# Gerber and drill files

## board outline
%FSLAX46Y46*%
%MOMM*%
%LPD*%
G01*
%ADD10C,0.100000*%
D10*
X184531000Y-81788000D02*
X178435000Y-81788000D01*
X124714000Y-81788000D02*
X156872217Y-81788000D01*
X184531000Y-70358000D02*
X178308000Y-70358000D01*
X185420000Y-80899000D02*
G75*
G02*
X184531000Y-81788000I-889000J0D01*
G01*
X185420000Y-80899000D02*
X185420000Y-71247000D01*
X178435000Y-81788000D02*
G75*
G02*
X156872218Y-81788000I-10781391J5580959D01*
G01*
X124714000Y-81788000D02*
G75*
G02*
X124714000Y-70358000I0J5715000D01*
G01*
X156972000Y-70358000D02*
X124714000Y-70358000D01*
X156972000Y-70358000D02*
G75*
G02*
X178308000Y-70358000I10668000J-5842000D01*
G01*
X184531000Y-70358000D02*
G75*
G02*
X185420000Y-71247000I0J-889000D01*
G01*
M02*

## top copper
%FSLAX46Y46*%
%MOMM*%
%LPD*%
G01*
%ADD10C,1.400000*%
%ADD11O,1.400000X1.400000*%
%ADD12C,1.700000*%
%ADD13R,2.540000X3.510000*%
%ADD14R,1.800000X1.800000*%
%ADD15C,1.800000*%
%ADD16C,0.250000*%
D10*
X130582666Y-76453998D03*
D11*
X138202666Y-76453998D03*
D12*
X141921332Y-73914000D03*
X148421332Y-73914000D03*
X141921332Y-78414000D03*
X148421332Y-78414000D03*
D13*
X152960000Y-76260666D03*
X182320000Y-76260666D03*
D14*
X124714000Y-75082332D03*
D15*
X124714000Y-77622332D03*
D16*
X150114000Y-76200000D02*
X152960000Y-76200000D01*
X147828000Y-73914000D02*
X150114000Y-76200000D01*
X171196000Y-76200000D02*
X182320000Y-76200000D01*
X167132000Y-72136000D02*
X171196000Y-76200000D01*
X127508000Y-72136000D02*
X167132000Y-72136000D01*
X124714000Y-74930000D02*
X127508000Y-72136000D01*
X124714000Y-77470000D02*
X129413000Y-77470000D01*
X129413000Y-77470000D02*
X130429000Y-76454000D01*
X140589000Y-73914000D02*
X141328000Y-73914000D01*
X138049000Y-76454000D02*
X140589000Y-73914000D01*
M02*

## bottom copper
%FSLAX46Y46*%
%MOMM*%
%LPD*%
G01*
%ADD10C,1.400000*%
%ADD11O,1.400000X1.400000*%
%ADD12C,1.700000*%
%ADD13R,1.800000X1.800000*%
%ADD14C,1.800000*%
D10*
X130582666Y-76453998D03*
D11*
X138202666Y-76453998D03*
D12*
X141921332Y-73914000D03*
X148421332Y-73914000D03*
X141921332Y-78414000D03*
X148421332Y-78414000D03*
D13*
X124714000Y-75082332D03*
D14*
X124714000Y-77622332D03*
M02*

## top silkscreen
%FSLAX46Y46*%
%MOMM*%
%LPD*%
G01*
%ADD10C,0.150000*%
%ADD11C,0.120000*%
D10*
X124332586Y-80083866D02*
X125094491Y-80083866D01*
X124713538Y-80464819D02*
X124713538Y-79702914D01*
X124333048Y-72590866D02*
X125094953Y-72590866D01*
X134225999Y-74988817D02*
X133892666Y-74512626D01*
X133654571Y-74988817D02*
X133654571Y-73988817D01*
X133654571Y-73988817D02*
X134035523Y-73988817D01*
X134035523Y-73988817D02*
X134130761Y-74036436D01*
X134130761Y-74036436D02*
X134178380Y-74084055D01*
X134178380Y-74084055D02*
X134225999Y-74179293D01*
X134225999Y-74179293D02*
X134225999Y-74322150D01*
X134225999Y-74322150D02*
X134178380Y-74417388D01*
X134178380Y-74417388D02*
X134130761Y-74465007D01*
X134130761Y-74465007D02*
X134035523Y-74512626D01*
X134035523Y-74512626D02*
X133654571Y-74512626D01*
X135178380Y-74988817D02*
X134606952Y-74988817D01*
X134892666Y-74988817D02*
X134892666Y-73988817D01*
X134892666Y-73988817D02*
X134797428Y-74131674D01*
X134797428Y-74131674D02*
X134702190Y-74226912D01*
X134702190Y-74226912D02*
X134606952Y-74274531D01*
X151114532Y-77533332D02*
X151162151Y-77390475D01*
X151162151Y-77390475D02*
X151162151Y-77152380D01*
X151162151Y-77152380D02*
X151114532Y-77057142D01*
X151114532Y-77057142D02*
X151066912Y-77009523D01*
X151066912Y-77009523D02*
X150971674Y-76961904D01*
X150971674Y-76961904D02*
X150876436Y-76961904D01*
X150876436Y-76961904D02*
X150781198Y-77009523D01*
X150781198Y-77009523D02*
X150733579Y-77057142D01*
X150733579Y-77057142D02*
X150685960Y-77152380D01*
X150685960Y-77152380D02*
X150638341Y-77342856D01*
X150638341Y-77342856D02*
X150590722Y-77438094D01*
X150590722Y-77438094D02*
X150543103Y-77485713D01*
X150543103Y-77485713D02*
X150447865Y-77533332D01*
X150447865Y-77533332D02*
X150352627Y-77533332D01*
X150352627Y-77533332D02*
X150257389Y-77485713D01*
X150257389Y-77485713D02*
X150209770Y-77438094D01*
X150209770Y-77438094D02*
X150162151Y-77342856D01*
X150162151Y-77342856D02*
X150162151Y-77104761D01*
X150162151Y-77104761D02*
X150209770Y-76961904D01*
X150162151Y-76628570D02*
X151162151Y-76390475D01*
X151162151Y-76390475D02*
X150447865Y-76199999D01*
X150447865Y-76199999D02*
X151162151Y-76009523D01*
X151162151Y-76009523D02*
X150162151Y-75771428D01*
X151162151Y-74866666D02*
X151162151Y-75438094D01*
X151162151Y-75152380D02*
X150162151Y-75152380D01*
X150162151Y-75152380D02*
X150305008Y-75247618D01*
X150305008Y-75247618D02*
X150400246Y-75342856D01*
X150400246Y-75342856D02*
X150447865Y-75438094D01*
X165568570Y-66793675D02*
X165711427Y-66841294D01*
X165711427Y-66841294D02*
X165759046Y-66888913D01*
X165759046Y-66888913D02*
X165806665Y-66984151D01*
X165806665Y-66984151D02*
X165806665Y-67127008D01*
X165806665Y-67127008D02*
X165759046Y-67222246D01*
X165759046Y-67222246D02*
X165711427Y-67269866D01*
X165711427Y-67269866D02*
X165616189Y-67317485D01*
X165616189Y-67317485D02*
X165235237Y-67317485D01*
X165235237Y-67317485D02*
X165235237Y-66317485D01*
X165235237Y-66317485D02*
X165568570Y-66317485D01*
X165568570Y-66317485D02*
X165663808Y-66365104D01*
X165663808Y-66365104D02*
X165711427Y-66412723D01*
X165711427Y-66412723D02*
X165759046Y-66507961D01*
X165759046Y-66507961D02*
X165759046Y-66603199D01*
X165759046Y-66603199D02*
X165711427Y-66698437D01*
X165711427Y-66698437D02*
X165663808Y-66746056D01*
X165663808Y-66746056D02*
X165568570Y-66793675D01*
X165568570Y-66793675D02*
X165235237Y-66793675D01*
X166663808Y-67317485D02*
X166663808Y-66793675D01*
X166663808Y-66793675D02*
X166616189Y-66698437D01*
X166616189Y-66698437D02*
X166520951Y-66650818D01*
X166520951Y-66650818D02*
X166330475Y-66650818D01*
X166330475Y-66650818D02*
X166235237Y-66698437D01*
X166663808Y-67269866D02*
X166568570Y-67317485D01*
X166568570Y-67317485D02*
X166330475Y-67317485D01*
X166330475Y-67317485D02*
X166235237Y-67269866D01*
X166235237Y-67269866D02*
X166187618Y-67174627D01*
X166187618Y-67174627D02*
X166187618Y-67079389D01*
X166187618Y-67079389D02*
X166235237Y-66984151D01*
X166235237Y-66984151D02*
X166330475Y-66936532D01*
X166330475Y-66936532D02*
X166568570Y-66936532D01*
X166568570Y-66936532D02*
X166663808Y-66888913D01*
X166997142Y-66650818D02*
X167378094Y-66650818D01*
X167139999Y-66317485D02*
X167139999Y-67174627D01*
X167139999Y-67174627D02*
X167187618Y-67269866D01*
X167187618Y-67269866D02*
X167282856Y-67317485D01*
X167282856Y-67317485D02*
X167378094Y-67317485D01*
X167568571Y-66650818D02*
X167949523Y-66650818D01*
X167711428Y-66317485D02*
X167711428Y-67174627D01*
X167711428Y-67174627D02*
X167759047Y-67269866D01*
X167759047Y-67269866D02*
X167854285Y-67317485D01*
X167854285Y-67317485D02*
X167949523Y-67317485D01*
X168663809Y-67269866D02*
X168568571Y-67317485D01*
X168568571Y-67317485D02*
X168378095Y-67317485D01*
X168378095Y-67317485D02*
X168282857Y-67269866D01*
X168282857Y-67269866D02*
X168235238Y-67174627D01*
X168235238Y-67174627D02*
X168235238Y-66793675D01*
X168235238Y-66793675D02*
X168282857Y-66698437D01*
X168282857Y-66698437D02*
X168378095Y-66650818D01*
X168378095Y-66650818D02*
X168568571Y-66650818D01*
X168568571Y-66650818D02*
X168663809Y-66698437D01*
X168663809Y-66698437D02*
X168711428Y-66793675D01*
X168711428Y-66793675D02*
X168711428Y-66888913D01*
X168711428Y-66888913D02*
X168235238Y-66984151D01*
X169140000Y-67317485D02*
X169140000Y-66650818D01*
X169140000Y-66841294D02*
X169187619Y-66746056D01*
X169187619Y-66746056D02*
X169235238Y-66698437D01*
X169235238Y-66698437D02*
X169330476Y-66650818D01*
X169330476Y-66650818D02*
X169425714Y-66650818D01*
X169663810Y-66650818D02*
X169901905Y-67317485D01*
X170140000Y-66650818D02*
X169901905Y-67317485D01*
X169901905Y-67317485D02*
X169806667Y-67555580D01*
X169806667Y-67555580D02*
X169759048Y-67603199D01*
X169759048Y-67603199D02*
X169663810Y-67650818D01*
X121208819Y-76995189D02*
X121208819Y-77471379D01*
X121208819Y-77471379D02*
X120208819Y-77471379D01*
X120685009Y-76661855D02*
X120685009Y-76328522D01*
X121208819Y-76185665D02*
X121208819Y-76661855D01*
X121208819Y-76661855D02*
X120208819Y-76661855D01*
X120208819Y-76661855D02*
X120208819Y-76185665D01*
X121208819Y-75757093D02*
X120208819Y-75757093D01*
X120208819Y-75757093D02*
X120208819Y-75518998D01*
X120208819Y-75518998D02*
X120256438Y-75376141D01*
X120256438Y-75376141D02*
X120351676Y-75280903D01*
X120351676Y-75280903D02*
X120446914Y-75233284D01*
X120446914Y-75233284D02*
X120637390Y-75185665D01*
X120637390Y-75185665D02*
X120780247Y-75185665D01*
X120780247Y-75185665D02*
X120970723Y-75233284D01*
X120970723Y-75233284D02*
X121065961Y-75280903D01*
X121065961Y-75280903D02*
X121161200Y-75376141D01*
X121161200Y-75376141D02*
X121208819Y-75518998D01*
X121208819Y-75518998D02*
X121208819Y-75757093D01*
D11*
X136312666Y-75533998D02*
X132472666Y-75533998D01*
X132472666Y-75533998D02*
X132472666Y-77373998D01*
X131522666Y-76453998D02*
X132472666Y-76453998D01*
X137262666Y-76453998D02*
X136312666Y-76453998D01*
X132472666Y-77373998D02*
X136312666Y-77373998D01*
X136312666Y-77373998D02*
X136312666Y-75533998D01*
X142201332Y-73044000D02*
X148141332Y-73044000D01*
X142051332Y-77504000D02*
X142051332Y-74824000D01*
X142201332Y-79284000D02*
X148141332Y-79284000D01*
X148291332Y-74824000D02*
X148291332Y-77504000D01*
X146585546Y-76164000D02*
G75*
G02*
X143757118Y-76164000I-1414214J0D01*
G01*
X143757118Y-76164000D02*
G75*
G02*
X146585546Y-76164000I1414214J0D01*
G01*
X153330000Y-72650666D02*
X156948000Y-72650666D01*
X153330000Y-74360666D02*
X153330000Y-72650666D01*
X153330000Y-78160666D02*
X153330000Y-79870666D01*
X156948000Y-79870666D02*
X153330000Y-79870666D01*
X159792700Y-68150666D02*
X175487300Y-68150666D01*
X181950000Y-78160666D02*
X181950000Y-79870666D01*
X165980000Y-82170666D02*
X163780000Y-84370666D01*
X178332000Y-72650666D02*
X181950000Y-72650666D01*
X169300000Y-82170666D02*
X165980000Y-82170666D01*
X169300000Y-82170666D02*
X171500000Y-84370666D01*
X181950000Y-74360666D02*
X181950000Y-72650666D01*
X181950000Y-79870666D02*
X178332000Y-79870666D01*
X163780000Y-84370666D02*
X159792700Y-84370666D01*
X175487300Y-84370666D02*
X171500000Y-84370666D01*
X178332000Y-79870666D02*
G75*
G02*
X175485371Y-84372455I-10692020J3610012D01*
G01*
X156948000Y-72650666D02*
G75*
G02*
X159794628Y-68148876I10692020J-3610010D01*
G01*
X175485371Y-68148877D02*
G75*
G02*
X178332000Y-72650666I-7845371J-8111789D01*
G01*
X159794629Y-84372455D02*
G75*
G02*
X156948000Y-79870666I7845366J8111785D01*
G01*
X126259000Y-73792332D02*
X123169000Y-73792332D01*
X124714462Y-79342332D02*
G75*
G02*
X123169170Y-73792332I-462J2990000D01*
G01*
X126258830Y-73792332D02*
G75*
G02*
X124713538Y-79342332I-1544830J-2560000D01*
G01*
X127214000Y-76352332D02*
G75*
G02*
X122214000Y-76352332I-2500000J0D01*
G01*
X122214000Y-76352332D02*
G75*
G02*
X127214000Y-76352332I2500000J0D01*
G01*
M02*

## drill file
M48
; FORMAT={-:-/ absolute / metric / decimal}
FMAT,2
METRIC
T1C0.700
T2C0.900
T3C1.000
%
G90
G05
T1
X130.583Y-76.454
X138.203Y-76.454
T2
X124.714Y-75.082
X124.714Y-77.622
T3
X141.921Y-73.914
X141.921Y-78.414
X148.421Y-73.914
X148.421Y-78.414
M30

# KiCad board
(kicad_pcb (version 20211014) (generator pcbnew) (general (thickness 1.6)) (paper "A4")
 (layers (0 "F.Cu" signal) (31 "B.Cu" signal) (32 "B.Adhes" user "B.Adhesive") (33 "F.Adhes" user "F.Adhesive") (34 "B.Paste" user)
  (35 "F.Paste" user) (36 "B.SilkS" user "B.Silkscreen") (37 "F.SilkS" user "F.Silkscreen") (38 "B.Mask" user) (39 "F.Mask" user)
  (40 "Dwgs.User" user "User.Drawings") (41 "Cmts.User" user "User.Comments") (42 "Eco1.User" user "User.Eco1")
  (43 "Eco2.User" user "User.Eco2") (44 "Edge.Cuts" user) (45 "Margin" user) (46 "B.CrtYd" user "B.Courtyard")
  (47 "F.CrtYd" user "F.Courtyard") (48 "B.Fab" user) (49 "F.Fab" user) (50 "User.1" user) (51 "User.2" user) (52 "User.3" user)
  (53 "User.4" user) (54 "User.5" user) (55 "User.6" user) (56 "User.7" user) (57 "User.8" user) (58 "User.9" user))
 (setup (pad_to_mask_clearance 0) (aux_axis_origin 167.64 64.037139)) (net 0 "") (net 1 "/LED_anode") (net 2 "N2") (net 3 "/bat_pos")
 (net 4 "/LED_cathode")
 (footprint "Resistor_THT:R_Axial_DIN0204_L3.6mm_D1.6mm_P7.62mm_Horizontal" (layer "F.Cu") (at 130.582666 76.453998)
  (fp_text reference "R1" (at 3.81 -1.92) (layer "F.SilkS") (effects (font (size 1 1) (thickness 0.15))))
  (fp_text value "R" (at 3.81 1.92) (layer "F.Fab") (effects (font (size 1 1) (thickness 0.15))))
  (fp_line (start 5.73 -0.92) (end 1.89 -0.92) (layer "F.SilkS") (width 0.12))
  (fp_line (start 1.89 -0.92) (end 1.89 0.92) (layer "F.SilkS") (width 0.12))
  (fp_line (start 0.94 0) (end 1.89 0) (layer "F.SilkS") (width 0.12))
  (fp_line (start 6.68 0) (end 5.73 0) (layer "F.SilkS") (width 0.12))
  (fp_line (start 1.89 0.92) (end 5.73 0.92) (layer "F.SilkS") (width 0.12))
  (fp_line (start 5.73 0.92) (end 5.73 -0.92) (layer "F.SilkS") (width 0.12))
  (pad "1" thru_hole circle (at 0 0) (size 1.4 1.4) (drill 0.7) (layers *.Cu *.Mask) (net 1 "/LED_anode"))
  (pad "2" thru_hole oval (at 7.62 0) (size 1.4 1.4) (drill 0.7) (layers *.Cu *.Mask) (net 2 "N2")))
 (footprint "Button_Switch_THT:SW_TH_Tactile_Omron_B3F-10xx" (layer "F.Cu") (at 141.921332 73.914)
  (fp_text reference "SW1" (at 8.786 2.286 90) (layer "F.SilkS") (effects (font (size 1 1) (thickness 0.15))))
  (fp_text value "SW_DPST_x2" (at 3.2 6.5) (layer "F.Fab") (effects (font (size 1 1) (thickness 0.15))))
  (fp_line (start 0.28 -0.87) (end 6.22 -0.87) (layer "F.SilkS") (width 0.12))
  (fp_line (start 0.13 3.59) (end 0.13 0.91) (layer "F.SilkS") (width 0.12))
  (fp_line (start 0.28 5.37) (end 6.22 5.37) (layer "F.SilkS") (width 0.12))
  (fp_line (start 6.37 0.91) (end 6.37 3.59) (layer "F.SilkS") (width 0.12))
  (fp_circle (center 3.25 2.25) (end 4.25 3.25) (layer "F.SilkS") (width 0.12) (fill none))
  (pad "1" thru_hole circle (at 0 0) (size 1.7 1.7) (drill 1) (layers *.Cu *.Mask) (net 2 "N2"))
  (pad "2" thru_hole circle (at 6.5 0) (size 1.7 1.7) (drill 1) (layers *.Cu *.Mask) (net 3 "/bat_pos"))
  (pad "3" thru_hole circle (at 0 4.5) (size 1.7 1.7) (drill 1) (layers *.Cu *.Mask))
  (pad "4" thru_hole circle (at 6.5 4.5) (size 1.7 1.7) (drill 1) (layers *.Cu *.Mask)))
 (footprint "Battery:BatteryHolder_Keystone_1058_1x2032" (layer "F.Cu") (at 167.64 76.260666)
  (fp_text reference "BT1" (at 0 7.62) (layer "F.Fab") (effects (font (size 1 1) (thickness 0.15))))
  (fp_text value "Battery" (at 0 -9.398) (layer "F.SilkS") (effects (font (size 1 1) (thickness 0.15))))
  (fp_line (start -14.31 -3.61) (end -10.692 -3.61) (layer "F.SilkS") (width 0.12))
  (fp_line (start -14.31 -1.9) (end -14.31 -3.61) (layer "F.SilkS") (width 0.12))
  (fp_line (start -14.31 1.9) (end -14.31 3.61) (layer "F.SilkS") (width 0.12))
  (fp_line (start -10.692 3.61) (end -14.31 3.61) (layer "F.SilkS") (width 0.12))
  (fp_line (start -7.8473 -8.11) (end 7.8473 -8.11) (layer "F.SilkS") (width 0.12))
  (fp_line (start 14.31 1.9) (end 14.31 3.61) (layer "F.SilkS") (width 0.12))
  (fp_line (start -1.66 5.91) (end -3.86 8.11) (layer "F.SilkS") (width 0.12))
  (fp_line (start 10.692 -3.61) (end 14.31 -3.61) (layer "F.SilkS") (width 0.12))
  (fp_line (start 1.66 5.91) (end -1.66 5.91) (layer "F.SilkS") (width 0.12))
  (fp_line (start 1.66 5.91) (end 3.86 8.11) (layer "F.SilkS") (width 0.12))
  (fp_line (start 14.31 -1.9) (end 14.31 -3.61) (layer "F.SilkS") (width 0.12))
  (fp_line (start 14.31 3.61) (end 10.692 3.61) (layer "F.SilkS") (width 0.12))
  (fp_line (start -3.86 8.11) (end -7.8473 8.11) (layer "F.SilkS") (width 0.12))
  (fp_line (start 7.8473 8.11) (end 3.86 8.11) (layer "F.SilkS") (width 0.12))
  (fp_arc (start 10.692 3.61) (mid 9.538084 6.031244) (end 7.845371 8.111789) (layer "F.SilkS") (width 0.12))
  (fp_arc (start -10.692 -3.61) (mid -9.538084 -6.031244) (end -7.845371 -8.111789) (layer "F.SilkS") (width 0.12))
  (fp_arc (start 7.845371 -8.111789) (mid 9.538085 -6.031244) (end 10.692 -3.61) (layer "F.SilkS") (width 0.12))
  (fp_arc (start -7.845371 8.111789) (mid -9.538085 6.031244) (end -10.692 3.61) (layer "F.SilkS") (width 0.12))
  (pad "1" smd rect (at -14.68 0) (size 2.54 3.51) (layers "F.Cu" "F.Paste" "F.Mask") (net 3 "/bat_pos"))
  (pad "2" smd rect (at 14.68 0) (size 2.54 3.51) (layers "F.Cu" "F.Paste" "F.Mask") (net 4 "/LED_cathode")))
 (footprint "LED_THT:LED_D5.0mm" (layer "F.Cu") (at 124.714 75.082332 -90)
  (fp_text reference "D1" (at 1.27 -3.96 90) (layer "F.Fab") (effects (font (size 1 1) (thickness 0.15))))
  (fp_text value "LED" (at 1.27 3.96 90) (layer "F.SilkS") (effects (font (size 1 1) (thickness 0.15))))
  (fp_line (start -1.29 -1.545) (end -1.29 1.545) (layer "F.SilkS") (width 0.12))
  (fp_arc (start 4.26 -0.000462) (mid 2.072002 2.880433) (end -1.29 1.54483) (layer "F.SilkS") (width 0.12))
  (fp_arc (start -1.29 -1.54483) (mid 2.072002 -2.880433) (end 4.26 0.000462) (layer "F.SilkS") (width 0.12))
  (fp_circle (center 1.27 0) (end 3.77 0) (layer "F.SilkS") (width 0.12) (fill none))
  (pad "1" thru_hole rect (at 0 0 270) (size 1.8 1.8) (drill 0.9) (layers *.Cu *.Mask) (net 4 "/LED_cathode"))
  (pad "2" thru_hole circle (at 2.54 0 270) (size 1.8 1.8) (drill 0.9) (layers *.Cu *.Mask) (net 1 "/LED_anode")))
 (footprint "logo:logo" (layer "B.Cu") (at 167.64 76.073 180)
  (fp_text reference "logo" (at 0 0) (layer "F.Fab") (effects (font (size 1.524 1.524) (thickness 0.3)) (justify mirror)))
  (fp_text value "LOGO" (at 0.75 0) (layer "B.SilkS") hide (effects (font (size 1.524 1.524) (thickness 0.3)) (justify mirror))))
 (gr_line (start 184.531 81.788) (end 178.435 81.788) (layer "Edge.Cuts") (width 0.1))
 (gr_line (start 124.714 81.788) (end 156.872217 81.788) (layer "Edge.Cuts") (width 0.1))
 (gr_line (start 184.531 70.358) (end 178.308 70.358) (layer "Edge.Cuts") (width 0.1))
 (gr_arc (start 185.42 80.899) (mid 185.159618 81.527618) (end 184.531 81.788) (layer "Edge.Cuts") (width 0.1))
 (gr_line (start 185.42 80.899) (end 185.42 71.247) (layer "Edge.Cuts") (width 0.1))
 (gr_arc (start 178.435 81.788) (mid 167.653609 88.347284) (end 156.872217 81.788) (layer "Edge.Cuts") (width 0.1))
 (gr_arc (start 124.714 81.788) (mid 118.999 76.073) (end 124.714 70.358) (layer "Edge.Cuts") (width 0.1))
 (gr_line (start 156.972 70.358) (end 124.714 70.358) (layer "Edge.Cuts") (width 0.1))
 (gr_arc (start 156.972 70.358) (mid 167.64 64.037139) (end 178.308 70.358) (layer "Edge.Cuts") (width 0.1))
 (gr_arc (start 184.531 70.358) (mid 185.159618 70.618382) (end 185.42 71.247) (layer "Edge.Cuts") (width 0.1))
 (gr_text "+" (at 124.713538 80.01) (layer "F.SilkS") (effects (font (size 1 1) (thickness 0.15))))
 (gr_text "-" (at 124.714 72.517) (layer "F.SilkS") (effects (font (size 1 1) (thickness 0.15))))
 (segment (start 150.114 76.2) (end 152.96 76.2) (width 0.25) (layer "F.Cu") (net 3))
 (segment (start 147.828 73.914) (end 150.114 76.2) (width 0.25) (layer "F.Cu") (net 3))
 (segment (start 171.196 76.2) (end 182.32 76.2) (width 0.25) (layer "F.Cu") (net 4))
 (segment (start 167.132 72.136) (end 171.196 76.2) (width 0.25) (layer "F.Cu") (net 4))
 (segment (start 127.508 72.136) (end 167.132 72.136) (width 0.25) (layer "F.Cu") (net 4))
 (segment (start 124.714 74.93) (end 127.508 72.136) (width 0.25) (layer "F.Cu") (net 4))
 (segment (start 124.714 77.47) (end 129.413 77.47) (width 0.25) (layer "F.Cu") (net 1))
 (segment (start 129.413 77.47) (end 130.429 76.454) (width 0.25) (layer "F.Cu") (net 1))
 (segment (start 140.589 73.914) (end 141.328 73.914) (width 0.25) (layer "F.Cu") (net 2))
 (segment (start 138.049 76.454) (end 140.589 73.914) (width 0.25) (layer "F.Cu") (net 2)))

